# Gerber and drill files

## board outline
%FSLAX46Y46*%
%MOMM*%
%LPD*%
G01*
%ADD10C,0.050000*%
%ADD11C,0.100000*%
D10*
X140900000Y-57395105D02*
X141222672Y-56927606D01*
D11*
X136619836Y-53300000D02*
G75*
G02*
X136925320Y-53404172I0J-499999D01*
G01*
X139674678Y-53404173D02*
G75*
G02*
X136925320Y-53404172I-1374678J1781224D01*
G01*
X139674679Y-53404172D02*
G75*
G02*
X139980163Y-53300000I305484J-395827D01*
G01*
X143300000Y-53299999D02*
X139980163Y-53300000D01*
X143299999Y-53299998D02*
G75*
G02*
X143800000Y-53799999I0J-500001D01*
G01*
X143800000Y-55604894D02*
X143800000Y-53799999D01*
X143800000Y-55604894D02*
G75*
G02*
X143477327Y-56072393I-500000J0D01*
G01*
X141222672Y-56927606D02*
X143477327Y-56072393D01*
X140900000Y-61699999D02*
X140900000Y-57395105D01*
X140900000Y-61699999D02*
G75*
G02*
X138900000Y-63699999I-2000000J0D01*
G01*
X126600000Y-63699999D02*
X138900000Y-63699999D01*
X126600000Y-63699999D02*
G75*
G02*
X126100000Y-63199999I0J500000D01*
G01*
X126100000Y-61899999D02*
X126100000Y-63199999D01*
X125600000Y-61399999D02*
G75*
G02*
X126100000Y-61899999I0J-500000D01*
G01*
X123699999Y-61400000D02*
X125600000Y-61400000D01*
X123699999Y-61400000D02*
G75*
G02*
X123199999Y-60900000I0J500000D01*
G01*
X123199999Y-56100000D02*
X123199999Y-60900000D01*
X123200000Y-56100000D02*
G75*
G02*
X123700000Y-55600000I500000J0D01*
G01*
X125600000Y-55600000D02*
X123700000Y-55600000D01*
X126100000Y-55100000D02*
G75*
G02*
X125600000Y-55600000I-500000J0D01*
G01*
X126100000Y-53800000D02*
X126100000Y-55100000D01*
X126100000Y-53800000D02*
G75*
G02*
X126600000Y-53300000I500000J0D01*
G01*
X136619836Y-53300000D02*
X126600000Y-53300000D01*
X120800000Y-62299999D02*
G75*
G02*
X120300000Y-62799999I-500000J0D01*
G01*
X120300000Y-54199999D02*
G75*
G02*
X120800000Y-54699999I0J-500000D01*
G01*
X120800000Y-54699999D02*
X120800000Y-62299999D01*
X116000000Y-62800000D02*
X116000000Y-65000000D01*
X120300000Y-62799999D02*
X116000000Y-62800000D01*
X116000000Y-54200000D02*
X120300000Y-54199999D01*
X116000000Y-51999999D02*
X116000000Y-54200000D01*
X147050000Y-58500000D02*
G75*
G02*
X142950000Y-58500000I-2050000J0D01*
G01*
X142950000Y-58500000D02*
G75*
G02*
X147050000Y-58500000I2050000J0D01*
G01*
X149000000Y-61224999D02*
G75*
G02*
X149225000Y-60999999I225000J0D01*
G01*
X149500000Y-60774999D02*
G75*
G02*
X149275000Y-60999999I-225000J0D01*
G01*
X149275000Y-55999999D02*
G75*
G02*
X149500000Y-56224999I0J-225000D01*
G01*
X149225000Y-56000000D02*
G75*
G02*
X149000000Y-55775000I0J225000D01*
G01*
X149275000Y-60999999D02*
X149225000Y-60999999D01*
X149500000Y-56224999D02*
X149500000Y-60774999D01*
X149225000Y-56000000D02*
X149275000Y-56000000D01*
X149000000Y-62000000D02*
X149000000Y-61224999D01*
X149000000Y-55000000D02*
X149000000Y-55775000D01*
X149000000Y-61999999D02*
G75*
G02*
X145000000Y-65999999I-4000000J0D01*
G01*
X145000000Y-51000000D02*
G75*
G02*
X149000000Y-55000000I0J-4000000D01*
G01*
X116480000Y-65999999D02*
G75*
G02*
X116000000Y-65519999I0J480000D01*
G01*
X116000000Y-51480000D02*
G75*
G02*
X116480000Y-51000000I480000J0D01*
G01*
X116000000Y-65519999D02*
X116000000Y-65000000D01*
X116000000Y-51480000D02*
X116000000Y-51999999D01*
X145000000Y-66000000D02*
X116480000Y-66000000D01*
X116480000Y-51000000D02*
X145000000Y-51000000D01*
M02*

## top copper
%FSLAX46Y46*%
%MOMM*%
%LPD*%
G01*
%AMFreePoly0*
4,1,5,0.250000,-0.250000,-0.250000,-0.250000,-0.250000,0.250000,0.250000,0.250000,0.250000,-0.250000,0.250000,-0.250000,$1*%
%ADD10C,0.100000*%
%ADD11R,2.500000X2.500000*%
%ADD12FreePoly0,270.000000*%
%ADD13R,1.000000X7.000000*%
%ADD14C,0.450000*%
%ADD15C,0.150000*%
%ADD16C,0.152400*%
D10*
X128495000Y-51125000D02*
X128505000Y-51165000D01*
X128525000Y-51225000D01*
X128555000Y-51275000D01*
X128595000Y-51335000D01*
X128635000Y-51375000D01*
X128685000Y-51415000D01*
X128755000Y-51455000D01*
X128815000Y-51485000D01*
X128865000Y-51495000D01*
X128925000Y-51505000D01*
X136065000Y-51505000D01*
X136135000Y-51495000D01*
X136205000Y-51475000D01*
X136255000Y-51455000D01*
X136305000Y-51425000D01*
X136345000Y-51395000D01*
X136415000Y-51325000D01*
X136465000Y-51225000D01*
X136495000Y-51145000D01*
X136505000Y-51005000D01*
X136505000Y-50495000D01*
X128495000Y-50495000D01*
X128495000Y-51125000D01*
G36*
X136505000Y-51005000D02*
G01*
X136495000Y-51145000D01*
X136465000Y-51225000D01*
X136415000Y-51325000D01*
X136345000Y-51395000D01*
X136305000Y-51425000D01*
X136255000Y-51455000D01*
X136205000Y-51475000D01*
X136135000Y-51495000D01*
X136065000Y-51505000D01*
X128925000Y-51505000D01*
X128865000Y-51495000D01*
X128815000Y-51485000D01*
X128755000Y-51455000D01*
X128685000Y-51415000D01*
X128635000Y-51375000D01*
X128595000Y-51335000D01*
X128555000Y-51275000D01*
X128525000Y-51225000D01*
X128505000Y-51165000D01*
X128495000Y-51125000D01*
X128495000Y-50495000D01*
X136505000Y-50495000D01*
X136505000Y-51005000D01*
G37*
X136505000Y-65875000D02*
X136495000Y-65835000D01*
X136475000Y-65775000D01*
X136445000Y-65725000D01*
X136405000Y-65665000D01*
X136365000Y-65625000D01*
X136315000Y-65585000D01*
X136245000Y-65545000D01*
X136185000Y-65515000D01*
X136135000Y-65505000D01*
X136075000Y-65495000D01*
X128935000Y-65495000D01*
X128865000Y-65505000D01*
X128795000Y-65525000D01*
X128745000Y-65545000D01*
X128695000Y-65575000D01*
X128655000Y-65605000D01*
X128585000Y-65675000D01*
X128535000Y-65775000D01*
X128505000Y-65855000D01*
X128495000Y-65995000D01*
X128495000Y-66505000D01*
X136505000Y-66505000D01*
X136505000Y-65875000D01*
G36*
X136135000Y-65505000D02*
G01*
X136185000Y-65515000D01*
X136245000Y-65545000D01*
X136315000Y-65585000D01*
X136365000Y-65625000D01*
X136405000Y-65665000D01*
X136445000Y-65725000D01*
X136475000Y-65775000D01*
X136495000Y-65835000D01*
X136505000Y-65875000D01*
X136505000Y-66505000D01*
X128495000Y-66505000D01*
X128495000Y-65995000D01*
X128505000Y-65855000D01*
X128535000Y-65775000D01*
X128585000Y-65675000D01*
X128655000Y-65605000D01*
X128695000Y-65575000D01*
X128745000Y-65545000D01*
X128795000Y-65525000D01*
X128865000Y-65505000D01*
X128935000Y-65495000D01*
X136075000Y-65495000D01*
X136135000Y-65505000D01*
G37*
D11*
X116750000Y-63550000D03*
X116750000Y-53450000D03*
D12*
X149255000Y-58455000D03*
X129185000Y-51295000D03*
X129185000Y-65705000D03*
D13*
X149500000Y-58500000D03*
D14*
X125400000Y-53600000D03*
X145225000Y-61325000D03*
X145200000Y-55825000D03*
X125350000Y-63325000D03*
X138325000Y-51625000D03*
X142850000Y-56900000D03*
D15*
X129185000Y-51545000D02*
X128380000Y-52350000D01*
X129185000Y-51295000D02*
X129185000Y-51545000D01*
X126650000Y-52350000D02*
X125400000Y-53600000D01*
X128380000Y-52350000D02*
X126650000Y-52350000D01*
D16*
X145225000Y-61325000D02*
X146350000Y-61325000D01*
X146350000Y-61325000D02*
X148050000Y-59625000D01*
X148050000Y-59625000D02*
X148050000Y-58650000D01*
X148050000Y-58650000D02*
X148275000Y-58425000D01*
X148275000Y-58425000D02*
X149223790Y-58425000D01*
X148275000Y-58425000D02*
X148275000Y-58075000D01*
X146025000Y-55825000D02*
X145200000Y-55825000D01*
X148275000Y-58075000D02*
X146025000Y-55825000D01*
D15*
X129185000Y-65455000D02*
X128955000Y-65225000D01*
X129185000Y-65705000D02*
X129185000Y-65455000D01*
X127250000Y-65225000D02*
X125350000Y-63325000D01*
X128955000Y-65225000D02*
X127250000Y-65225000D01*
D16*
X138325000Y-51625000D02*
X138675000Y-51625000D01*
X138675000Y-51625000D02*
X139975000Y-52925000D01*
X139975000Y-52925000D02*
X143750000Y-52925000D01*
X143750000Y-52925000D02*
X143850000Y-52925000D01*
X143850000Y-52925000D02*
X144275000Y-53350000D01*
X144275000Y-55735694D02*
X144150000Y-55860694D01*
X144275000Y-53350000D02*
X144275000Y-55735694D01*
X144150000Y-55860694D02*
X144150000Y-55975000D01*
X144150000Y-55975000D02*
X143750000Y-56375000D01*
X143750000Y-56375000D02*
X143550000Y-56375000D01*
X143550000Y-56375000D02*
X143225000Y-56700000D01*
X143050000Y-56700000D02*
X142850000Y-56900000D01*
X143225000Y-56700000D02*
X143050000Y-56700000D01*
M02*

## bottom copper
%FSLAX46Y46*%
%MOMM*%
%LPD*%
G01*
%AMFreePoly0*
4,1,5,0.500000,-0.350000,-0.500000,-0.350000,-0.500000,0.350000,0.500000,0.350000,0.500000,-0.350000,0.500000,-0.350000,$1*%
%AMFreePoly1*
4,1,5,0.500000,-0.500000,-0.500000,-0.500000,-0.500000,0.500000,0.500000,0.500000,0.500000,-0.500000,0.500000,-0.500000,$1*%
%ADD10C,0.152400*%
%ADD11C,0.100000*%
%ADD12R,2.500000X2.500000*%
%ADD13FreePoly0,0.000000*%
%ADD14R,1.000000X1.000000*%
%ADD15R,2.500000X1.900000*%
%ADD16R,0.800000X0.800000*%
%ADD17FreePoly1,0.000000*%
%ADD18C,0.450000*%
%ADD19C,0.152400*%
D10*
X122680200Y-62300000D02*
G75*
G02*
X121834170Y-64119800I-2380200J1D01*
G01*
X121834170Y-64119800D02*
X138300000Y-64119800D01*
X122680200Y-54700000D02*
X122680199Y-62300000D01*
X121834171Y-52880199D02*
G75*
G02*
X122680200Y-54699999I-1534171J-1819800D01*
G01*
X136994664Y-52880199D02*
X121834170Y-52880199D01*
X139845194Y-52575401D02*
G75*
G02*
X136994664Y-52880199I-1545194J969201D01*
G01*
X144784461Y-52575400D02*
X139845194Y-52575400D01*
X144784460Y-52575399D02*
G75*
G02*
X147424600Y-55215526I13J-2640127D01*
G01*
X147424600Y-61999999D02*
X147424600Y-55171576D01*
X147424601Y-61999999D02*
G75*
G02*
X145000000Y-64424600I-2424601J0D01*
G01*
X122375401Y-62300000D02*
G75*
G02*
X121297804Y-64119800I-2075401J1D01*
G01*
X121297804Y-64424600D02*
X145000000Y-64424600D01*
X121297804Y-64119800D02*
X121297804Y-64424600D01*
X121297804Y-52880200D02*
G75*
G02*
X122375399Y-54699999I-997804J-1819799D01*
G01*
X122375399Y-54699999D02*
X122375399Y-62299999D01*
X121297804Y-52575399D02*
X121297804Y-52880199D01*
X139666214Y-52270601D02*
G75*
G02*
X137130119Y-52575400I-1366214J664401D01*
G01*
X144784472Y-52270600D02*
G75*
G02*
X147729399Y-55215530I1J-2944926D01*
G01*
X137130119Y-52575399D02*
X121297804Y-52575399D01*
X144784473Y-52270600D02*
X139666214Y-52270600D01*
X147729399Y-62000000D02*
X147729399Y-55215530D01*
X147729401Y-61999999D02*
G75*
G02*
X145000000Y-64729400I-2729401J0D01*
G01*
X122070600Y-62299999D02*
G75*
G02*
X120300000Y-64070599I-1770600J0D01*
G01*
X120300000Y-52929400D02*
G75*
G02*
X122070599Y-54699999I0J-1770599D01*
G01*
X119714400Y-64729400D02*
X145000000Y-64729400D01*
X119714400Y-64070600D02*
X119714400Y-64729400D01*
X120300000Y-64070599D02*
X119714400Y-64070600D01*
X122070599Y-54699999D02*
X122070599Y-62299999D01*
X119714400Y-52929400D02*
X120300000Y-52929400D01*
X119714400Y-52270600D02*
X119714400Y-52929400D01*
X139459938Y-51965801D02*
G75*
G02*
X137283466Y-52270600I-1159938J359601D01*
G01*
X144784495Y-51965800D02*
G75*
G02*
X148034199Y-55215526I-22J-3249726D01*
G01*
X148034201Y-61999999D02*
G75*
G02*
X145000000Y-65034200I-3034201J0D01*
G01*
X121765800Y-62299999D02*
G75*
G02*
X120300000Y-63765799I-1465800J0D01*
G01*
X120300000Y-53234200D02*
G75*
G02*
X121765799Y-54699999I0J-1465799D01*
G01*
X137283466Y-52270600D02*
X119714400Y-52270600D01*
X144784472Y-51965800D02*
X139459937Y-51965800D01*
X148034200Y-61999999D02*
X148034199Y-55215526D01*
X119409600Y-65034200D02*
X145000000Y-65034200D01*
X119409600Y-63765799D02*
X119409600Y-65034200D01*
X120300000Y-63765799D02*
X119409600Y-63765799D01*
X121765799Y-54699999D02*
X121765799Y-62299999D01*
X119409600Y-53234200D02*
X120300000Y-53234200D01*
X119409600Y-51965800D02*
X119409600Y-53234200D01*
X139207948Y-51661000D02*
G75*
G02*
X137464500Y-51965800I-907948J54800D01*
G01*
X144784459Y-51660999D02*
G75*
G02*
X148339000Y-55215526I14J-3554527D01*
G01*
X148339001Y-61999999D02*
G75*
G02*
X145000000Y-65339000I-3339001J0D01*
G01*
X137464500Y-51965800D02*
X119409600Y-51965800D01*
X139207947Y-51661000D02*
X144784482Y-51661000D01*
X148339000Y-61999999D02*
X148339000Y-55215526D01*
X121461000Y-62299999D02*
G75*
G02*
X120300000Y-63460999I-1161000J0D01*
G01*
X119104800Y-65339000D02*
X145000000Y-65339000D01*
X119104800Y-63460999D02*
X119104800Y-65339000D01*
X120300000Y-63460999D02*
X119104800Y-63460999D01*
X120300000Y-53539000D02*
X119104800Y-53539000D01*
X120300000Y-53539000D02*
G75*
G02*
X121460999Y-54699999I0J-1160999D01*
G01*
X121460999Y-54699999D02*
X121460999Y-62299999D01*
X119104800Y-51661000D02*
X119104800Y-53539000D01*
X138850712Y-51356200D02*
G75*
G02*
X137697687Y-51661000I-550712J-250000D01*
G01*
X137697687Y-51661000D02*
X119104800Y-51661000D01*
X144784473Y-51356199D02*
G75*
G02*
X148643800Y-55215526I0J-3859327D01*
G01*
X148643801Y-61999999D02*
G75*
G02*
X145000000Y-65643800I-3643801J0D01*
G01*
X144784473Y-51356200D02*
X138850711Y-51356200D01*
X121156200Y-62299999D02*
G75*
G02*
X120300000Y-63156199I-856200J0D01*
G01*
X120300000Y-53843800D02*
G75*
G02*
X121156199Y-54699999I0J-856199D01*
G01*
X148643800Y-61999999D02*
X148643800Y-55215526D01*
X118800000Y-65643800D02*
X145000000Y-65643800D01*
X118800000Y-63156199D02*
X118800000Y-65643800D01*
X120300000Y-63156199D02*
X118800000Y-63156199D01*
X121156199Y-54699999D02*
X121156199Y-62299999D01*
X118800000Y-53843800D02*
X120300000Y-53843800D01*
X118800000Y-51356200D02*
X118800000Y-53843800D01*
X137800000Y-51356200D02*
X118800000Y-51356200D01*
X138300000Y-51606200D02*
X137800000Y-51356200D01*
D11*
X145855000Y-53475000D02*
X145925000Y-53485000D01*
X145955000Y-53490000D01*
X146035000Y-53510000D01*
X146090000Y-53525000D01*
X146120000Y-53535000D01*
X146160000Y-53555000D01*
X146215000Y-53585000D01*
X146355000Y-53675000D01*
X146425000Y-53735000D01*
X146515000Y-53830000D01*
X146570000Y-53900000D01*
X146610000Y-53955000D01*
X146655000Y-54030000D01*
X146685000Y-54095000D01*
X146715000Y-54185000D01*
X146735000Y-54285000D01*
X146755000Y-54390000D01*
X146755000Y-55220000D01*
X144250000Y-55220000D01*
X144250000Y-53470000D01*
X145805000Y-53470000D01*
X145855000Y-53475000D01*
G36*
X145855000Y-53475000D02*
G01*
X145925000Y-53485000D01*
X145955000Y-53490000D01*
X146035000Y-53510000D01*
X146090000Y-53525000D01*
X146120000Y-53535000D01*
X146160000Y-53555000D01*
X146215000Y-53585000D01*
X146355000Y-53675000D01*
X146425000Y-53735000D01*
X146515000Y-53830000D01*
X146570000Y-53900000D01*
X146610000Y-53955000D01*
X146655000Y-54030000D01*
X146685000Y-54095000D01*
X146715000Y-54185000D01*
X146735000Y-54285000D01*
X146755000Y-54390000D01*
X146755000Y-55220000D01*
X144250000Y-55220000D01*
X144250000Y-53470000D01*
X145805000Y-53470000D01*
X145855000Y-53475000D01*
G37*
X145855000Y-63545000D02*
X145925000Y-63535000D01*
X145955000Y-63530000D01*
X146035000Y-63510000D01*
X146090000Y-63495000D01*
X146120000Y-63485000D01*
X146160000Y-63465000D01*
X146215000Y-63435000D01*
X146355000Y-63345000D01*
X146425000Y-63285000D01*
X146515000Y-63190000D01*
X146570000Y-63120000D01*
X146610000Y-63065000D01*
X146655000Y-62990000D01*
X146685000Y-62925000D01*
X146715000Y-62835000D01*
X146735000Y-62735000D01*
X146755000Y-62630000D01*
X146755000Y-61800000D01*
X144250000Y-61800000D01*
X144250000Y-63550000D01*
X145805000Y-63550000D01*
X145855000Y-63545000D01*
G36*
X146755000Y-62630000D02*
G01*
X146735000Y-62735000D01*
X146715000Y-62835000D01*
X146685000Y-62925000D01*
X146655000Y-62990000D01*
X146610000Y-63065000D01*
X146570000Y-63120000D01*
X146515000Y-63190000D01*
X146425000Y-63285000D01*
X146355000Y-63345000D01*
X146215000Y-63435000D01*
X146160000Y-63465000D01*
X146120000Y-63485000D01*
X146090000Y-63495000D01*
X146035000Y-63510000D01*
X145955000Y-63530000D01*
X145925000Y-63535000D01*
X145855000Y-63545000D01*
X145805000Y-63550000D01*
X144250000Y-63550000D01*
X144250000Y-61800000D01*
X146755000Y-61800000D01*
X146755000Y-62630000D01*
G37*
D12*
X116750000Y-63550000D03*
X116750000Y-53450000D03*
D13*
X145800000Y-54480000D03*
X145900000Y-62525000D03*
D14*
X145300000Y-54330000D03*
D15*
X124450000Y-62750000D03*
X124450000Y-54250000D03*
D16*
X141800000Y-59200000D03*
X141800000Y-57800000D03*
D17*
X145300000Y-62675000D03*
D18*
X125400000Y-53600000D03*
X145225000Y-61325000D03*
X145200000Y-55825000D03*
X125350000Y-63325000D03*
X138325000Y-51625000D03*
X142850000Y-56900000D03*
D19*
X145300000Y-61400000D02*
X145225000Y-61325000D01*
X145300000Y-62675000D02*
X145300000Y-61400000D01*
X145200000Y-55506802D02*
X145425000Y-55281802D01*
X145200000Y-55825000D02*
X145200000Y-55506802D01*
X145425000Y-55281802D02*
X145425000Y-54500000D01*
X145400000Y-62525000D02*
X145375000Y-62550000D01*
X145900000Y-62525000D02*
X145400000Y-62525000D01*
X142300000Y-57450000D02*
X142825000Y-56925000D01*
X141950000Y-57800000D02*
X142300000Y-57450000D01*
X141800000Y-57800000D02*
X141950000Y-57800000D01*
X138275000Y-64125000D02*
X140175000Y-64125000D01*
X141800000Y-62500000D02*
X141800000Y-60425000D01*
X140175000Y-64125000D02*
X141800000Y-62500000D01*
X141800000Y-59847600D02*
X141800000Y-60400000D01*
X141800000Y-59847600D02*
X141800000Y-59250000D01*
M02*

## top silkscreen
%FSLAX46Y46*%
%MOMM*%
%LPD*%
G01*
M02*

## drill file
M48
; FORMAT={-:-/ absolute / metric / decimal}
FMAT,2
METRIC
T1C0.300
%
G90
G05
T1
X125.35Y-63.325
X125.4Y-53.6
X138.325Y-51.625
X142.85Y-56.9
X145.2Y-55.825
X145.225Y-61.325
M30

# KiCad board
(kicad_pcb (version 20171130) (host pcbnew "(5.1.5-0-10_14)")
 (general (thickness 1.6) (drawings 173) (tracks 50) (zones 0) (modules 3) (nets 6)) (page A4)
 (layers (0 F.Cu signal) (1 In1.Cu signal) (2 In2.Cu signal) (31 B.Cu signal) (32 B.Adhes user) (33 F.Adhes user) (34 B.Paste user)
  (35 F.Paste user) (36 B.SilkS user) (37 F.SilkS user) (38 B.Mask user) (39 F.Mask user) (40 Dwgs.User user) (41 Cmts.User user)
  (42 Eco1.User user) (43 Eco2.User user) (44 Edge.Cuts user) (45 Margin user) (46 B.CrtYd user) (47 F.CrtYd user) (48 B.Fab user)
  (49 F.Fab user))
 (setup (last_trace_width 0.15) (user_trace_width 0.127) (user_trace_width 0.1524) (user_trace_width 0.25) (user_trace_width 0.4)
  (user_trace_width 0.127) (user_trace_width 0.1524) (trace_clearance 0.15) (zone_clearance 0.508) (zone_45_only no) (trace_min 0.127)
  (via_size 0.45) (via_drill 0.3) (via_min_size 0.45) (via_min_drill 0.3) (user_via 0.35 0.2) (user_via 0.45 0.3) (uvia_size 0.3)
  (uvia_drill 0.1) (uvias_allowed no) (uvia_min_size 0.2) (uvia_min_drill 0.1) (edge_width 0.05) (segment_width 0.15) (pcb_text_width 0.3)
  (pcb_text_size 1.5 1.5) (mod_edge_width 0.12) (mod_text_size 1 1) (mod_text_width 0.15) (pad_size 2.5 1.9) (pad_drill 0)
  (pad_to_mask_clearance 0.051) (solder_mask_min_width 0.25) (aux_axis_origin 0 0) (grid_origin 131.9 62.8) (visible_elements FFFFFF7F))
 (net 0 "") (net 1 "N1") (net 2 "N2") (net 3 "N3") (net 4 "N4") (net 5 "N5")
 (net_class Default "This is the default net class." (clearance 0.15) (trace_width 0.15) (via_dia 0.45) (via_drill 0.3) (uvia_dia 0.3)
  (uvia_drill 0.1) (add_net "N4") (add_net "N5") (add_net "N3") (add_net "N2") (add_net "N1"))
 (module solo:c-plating (layer F.Cu) (at 116.9 53.35)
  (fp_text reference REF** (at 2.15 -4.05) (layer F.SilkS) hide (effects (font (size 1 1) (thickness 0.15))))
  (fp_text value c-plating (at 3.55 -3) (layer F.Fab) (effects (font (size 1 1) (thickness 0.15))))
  (pad 1 smd rect (at -0.15 10.2) (size 2.5 2.5) (layers B.Cu B.Mask))
  (pad 1 smd rect (at -0.15 0.1) (size 2.5 2.5) (layers B.Cu B.Mask))
  (pad 2 smd rect (at -0.15 10.2) (size 2.5 2.5) (layers F.Cu F.Mask))
  (pad 1 smd rect (at -0.15 0.1) (size 2.5 2.5) (layers F.Cu F.Mask)))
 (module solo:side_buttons (layer B.Cu) (at 149.525 58.075)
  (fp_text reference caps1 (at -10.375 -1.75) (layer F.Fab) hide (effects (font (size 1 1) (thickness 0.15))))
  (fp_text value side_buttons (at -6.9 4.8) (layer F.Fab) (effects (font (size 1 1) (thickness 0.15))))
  (fp_poly
   (pts (xy -21.03 -6.95) (xy -21.02 -6.91) (xy -21 -6.85) (xy -20.97 -6.8) (xy -20.93 -6.74) (xy -20.89 -6.7) (xy -20.84 -6.66)
    (xy -20.77 -6.62) (xy -20.71 -6.59) (xy -20.66 -6.58) (xy -20.6 -6.57) (xy -13.46 -6.57) (xy -13.39 -6.58) (xy -13.32 -6.6)
    (xy -13.27 -6.62) (xy -13.22 -6.65) (xy -13.18 -6.68) (xy -13.11 -6.75) (xy -13.06 -6.85) (xy -13.03 -6.93) (xy -13.02 -7.07)
    (xy -13.02 -7.58) (xy -21.03 -7.58))
   (layer F.Cu) (width 0.1))
  (fp_poly
   (pts (xy -13.02 7.8) (xy -13.03 7.76) (xy -13.05 7.7) (xy -13.08 7.65) (xy -13.12 7.59) (xy -13.16 7.55) (xy -13.21 7.51)
    (xy -13.28 7.47) (xy -13.34 7.44) (xy -13.39 7.43) (xy -13.45 7.42) (xy -20.59 7.42) (xy -20.66 7.43) (xy -20.73 7.45) (xy -20.78 7.47)
    (xy -20.83 7.5) (xy -20.87 7.53) (xy -20.94 7.6) (xy -20.99 7.7) (xy -21.02 7.78) (xy -21.03 7.92) (xy -21.03 8.43) (xy -13.02 8.43))
   (layer F.Cu) (width 0.1))
  (pad 3 smd custom (at -0.27 0.38 270) (size 0.5 0.5) (layers F.Cu) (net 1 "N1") (solder_mask_margin 0.01) (zone_connect 0)
   (options (clearance outline) (anchor rect)) (primitives))
  (pad 2 smd custom (at -20.34 -6.78 270) (size 0.5 0.5) (layers F.Cu) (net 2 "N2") (solder_mask_margin 0.01) (zone_connect 0)
   (options (clearance outline) (anchor rect)) (primitives))
  (pad 1 smd custom (at -20.34 7.63 270) (size 0.5 0.5) (layers F.Cu) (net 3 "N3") (solder_mask_margin 0.01) (zone_connect 0)
   (options (clearance outline) (anchor rect)) (primitives))
  (pad 3 smd rect (at -0.025 0.425 270) (size 7 1) (layers F.Cu F.Mask) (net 1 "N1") (solder_mask_margin 0.01)))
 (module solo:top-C (layer B.Cu) (at 114.8 58.375)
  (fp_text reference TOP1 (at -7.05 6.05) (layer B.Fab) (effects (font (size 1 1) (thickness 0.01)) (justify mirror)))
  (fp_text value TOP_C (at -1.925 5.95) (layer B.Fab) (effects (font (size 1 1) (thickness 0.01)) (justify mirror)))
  (fp_poly
   (pts (xy 31.055 -4.9) (xy 31.125 -4.89) (xy 31.155 -4.885) (xy 31.235 -4.865) (xy 31.29 -4.85) (xy 31.32 -4.84) (xy 31.36 -4.82)
    (xy 31.415 -4.79) (xy 31.555 -4.7) (xy 31.625 -4.64) (xy 31.715 -4.545) (xy 31.77 -4.475) (xy 31.81 -4.42) (xy 31.855 -4.345)
    (xy 31.885 -4.28) (xy 31.915 -4.19) (xy 31.935 -4.09) (xy 31.955 -3.985) (xy 31.955 -3.155) (xy 29.45 -3.155) (xy 29.45 -4.905)
    (xy 31.005 -4.905))
   (layer B.Cu) (width 0.1))
  (fp_poly
   (pts (xy 31.055 5.17) (xy 31.125 5.16) (xy 31.155 5.155) (xy 31.235 5.135) (xy 31.29 5.12) (xy 31.32 5.11) (xy 31.36 5.09)
    (xy 31.415 5.06) (xy 31.555 4.97) (xy 31.625 4.91) (xy 31.715 4.815) (xy 31.77 4.745) (xy 31.81 4.69) (xy 31.855 4.615) (xy 31.885 4.55)
    (xy 31.915 4.46) (xy 31.935 4.36) (xy 31.955 4.255) (xy 31.955 3.425) (xy 29.45 3.425) (xy 29.45 5.175) (xy 31.005 5.175))
   (layer B.Cu) (width 0.1))
  (pad 9 smd custom (at 31 -3.895) (size 1 0.7) (layers B.Cu B.Paste B.Mask) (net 1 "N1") (solder_paste_margin_ratio -0.05) (zone_connect 0)
   (options (clearance outline) (anchor rect)) (primitives))
  (pad 9 smd custom (at 31.1 4.15) (size 1 0.7) (layers B.Cu B.Paste B.Mask) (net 1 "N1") (solder_paste_margin_ratio -0.05) (zone_connect 0)
   (options (clearance outline) (anchor rect)) (primitives))
  (pad 9 smd rect (at 30.5 -4.045) (size 1 1) (layers B.Cu B.Paste B.Mask) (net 1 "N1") (solder_paste_margin_ratio -0.05))
  (pad 5 smd rect (at 9.65 4.375) (size 2.5 1.9) (layers B.Cu B.Paste B.Mask) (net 3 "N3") (solder_paste_margin_ratio -0.25))
  (pad 6 smd rect (at 9.65 -4.125) (size 2.5 1.9) (layers B.Cu B.Paste B.Mask) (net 2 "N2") (solder_paste_margin_ratio -0.25))
  (pad 7 smd rect (at 27 0.825) (size 0.8 0.8) (layers B.Cu B.Paste B.Mask) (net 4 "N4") (solder_paste_margin_ratio -0.2))
  (pad 8 smd rect (at 27 -0.575) (size 0.8 0.8) (layers B.Cu B.Paste B.Mask) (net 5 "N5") (solder_paste_margin_ratio -0.2))
  (pad 9 smd custom (at 30.5 4.3) (size 1 1) (layers B.Cu B.Paste B.Mask) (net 1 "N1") (solder_paste_margin_ratio -0.05) (zone_connect 0)
   (options (clearance outline) (anchor rect)) (primitives)))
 (gr_line (start 140.9 57.395105) (end 141.222672 56.927606) (layer Edge.Cuts) (width 0.05))
 (gr_arc (start 120.3 62.299999) (end 121.83417 64.1198) (angle -49.86765021) (layer B.Cu) (width 0.1524))
 (gr_line (start 121.83417 64.1198) (end 138.3 64.1198) (layer B.Cu) (width 0.1524))
 (gr_line (start 122.6802 54.7) (end 122.680199 62.3) (layer B.Cu) (width 0.1524))
 (gr_arc (start 120.3 54.699999) (end 122.6802 54.699999) (angle -49.86765021) (layer B.Cu) (width 0.1524))
 (gr_line (start 136.994664 52.880199) (end 121.83417 52.880199) (layer B.Cu) (width 0.1524))
 (gr_arc (start 138.3 51.6062) (end 136.994664 52.880199) (angle -103.59866) (layer B.Cu) (width 0.1524))
 (gr_line (start 144.784461 52.5754) (end 139.845194 52.5754) (layer B.Cu) (width 0.1524))
 (gr_arc (start 144.784473 55.215526) (end 147.4246 55.215526) (angle -90.00027385) (layer B.Cu) (width 0.1524))
 (gr_line (start 147.4246 61.999999) (end 147.4246 55.171576) (layer B.Cu) (width 0.1524))
 (gr_arc (start 145 61.999999) (end 145 64.4246) (angle -90) (layer B.Cu) (width 0.1524))
 (gr_arc (start 120.3 62.299999) (end 121.297804 64.1198) (angle -61.26385234) (layer B.Cu) (width 0.1524))
 (gr_line (start 121.297804 64.4246) (end 145 64.4246) (layer B.Cu) (width 0.1524))
 (gr_line (start 121.297804 64.1198) (end 121.297804 64.4246) (layer B.Cu) (width 0.1524))
 (gr_arc (start 120.3 54.699999) (end 122.375399 54.699999) (angle -61.26385234) (layer B.Cu) (width 0.1524))
 (gr_line (start 122.375399 54.699999) (end 122.375399 62.299999) (layer B.Cu) (width 0.1524))
 (gr_line (start 121.297804 52.575399) (end 121.297804 52.880199) (layer B.Cu) (width 0.1524))
 (gr_arc (start 138.3 51.6062) (end 137.130119 52.5754) (angle -114.4255887) (layer B.Cu) (width 0.1524))
 (gr_arc (start 144.784473 55.215526) (end 147.729399 55.21553) (angle -90.0000935) (layer B.Cu) (width 0.1524))
 (gr_line (start 137.130119 52.575399) (end 121.297804 52.575399) (layer B.Cu) (width 0.1524))
 (gr_line (start 144.784473 52.2706) (end 139.666214 52.2706) (layer B.Cu) (width 0.1524))
 (gr_line (start 147.729399 62) (end 147.729399 55.21553) (layer B.Cu) (width 0.1524))
 (gr_arc (start 145 61.999999) (end 145 64.7294) (angle -90) (layer B.Cu) (width 0.1524))
 (gr_arc (start 120.3 62.299999) (end 120.3 64.070599) (angle -89.99998951) (layer B.Cu) (width 0.1524))
 (gr_arc (start 120.3 54.699999) (end 122.070599 54.699999) (angle -90) (layer B.Cu) (width 0.1524))
 (gr_line (start 119.7144 64.7294) (end 145 64.7294) (layer B.Cu) (width 0.1524))
 (gr_line (start 119.7144 64.0706) (end 119.7144 64.7294) (layer B.Cu) (width 0.1524))
 (gr_line (start 120.3 64.070599) (end 119.7144 64.0706) (layer B.Cu) (width 0.1524))
 (gr_line (start 122.070599 54.699999) (end 122.070599 62.299999) (layer B.Cu) (width 0.1524))
 (gr_line (start 119.7144 52.9294) (end 120.3 52.9294) (layer B.Cu) (width 0.1524))
 (gr_line (start 119.7144 52.2706) (end 119.7144 52.9294) (layer B.Cu) (width 0.1524))
 (gr_arc (start 138.3 51.6062) (end 137.283466 52.2706) (angle -129.6073052) (layer B.Cu) (width 0.1524))
 (gr_arc (start 144.784473 55.215526) (end 148.034199 55.215526) (angle -89.99961615) (layer B.Cu) (width 0.1524))
 (gr_arc (start 145 61.999999) (end 145 65.0342) (angle -90) (layer B.Cu) (width 0.1524))
 (gr_arc (start 120.3 62.299999) (end 120.3 63.765799) (angle -90) (layer B.Cu) (width 0.1524))
 (gr_arc (start 120.3 54.699999) (end 121.765799 54.699999) (angle -90) (layer B.Cu) (width 0.1524))
 (gr_line (start 137.283466 52.2706) (end 119.7144 52.2706) (layer B.Cu) (width 0.1524))
 (gr_line (start 144.784472 51.9658) (end 139.459937 51.9658) (layer B.Cu) (width 0.1524))
 (gr_line (start 148.0342 61.999999) (end 148.034199 55.215526) (layer B.Cu) (width 0.1524))
 (gr_line (start 119.4096 65.0342) (end 145 65.0342) (layer B.Cu) (width 0.1524))
 (gr_line (start 119.4096 63.765799) (end 119.4096 65.0342) (layer B.Cu) (width 0.1524))
 (gr_line (start 120.3 63.765799) (end 119.4096 63.765799) (layer B.Cu) (width 0.1524))
 (gr_line (start 121.765799 54.699999) (end 121.765799 62.299999) (layer B.Cu) (width 0.1524))
 (gr_line (start 119.4096 53.2342) (end 120.3 53.2342) (layer B.Cu) (width 0.1524))
 (gr_line (start 119.4096 51.9658) (end 119.4096 53.2342) (layer B.Cu) (width 0.1524))
 (gr_arc (start 138.3 51.6062) (end 137.4645 51.9658) (angle -153.2589579) (layer B.Cu) (width 0.1524))
 (gr_arc (start 144.784473 55.215526) (end 148.339 55.215526) (angle -90.00022865) (layer B.Cu) (width 0.1524))
 (gr_arc (start 145 61.999999) (end 145 65.339) (angle -90) (layer B.Cu) (width 0.1524))
 (gr_line (start 137.4645 51.9658) (end 119.4096 51.9658) (layer B.Cu) (width 0.1524))
 (gr_line (start 139.207947 51.661) (end 144.784482 51.661) (layer B.Cu) (width 0.1524))
 (gr_line (start 148.339 61.999999) (end 148.339 55.215526) (layer B.Cu) (width 0.1524))
 (gr_arc (start 120.3 62.299999) (end 120.3 63.460999) (angle -90) (layer B.Cu) (width 0.1524))
 (gr_line (start 119.1048 65.339) (end 145 65.339) (layer B.Cu) (width 0.1524))
 (gr_line (start 119.1048 63.460999) (end 119.1048 65.339) (layer B.Cu) (width 0.1524))
 (gr_line (start 120.3 63.460999) (end 119.1048 63.460999) (layer B.Cu) (width 0.1524))
 (gr_line (start 120.3 53.539) (end 119.1048 53.539) (layer B.Cu) (width 0.1524))
 (gr_arc (start 120.3 54.699999) (end 121.460999 54.699999) (angle -90) (layer B.Cu) (width 0.1524))
 (gr_line (start 121.460999 54.699999) (end 121.460999 62.299999) (layer B.Cu) (width 0.1524))
 (gr_line (start 119.1048 51.661) (end 119.1048 53.539) (layer B.Cu) (width 0.1524))
 (gr_arc (start 138.3 51.6062) (end 137.697687 51.661) (angle -199.2174543) (layer B.Cu) (width 0.1524))
 (gr_line (start 137.697687 51.661) (end 119.1048 51.661) (layer B.Cu) (width 0.1524))
 (gr_arc (start 144.784473 55.215526) (end 148.6438 55.215526) (angle -90) (layer B.Cu) (width 0.1524))
 (gr_arc (start 145 61.999999) (end 145 65.6438) (angle -90) (layer B.Cu) (width 0.1524))
 (gr_line (start 144.784473 51.3562) (end 138.850711 51.3562) (layer B.Cu) (width 0.1524))
 (gr_arc (start 120.3 62.299999) (end 120.3 63.156199) (angle -90) (layer B.Cu) (width 0.1524))
 (gr_arc (start 120.3 54.699999) (end 121.156199 54.699999) (angle -90) (layer B.Cu) (width 0.1524))
 (gr_line (start 148.6438 61.999999) (end 148.6438 55.215526) (layer B.Cu) (width 0.1524))
 (gr_line (start 118.8 65.6438) (end 145 65.6438) (layer B.Cu) (width 0.1524))
 (gr_line (start 118.8 63.156199) (end 118.8 65.6438) (layer B.Cu) (width 0.1524))
 (gr_line (start 120.3 63.156199) (end 118.8 63.156199) (layer B.Cu) (width 0.1524))
 (gr_line (start 121.156199 54.699999) (end 121.156199 62.299999) (layer B.Cu) (width 0.1524))
 (gr_line (start 118.8 53.8438) (end 120.3 53.8438) (layer B.Cu) (width 0.1524))
 (gr_line (start 118.8 51.3562) (end 118.8 53.8438) (layer B.Cu) (width 0.1524))
 (gr_line (start 137.8 51.3562) (end 118.8 51.3562) (layer B.Cu) (width 0.1524))
 (gr_line (start 138.3 51.6062) (end 137.8 51.3562) (layer B.Cu) (width 0.1524))
 (gr_arc (start 136.619836 53.799999) (end 136.92532 53.404172) (angle -37.6595652) (layer Edge.Cuts) (width 0.1))
 (gr_arc (start 138.3 51.622949) (end 136.92532 53.404172) (angle -75.31913041) (layer Edge.Cuts) (width 0.1))
 (gr_arc (start 139.980163 53.799999) (end 139.980163 53.3) (angle -37.6595652) (layer Edge.Cuts) (width 0.1))
 (gr_line (start 143.3 53.299999) (end 139.980163 53.3) (layer Edge.Cuts) (width 0.1))
 (gr_arc (start 143.299999 53.799999) (end 143.8 53.799999) (angle -90) (layer Edge.Cuts) (width 0.1))
 (gr_line (start 143.8 55.604894) (end 143.8 53.799999) (layer Edge.Cuts) (width 0.1))
 (gr_arc (start 143.3 55.604894) (end 143.477327 56.072393) (angle -69.22774532) (layer Edge.Cuts) (width 0.1))
 (gr_line (start 141.222672 56.927606) (end 143.477327 56.072393) (layer Edge.Cuts) (width 0.1))
 (gr_line (start 140.9 61.699999) (end 140.9 57.395105) (layer Edge.Cuts) (width 0.1))
 (gr_arc (start 138.9 61.699999) (end 138.9 63.699999) (angle -90) (layer Edge.Cuts) (width 0.1))
 (gr_line (start 126.6 63.699999) (end 138.9 63.699999) (layer Edge.Cuts) (width 0.1))
 (gr_arc (start 126.6 63.199999) (end 126.1 63.199999) (angle -90) (layer Edge.Cuts) (width 0.1))
 (gr_line (start 126.1 61.899999) (end 126.1 63.199999) (layer Edge.Cuts) (width 0.1))
 (gr_arc (start 125.6 61.899999) (end 126.1 61.899999) (angle -90) (layer Edge.Cuts) (width 0.1))
 (gr_line (start 123.699999 61.4) (end 125.6 61.4) (layer Edge.Cuts) (width 0.1))
 (gr_arc (start 123.699999 60.9) (end 123.199999 60.9) (angle -90) (layer Edge.Cuts) (width 0.1))
 (gr_line (start 123.199999 56.1) (end 123.199999 60.9) (layer Edge.Cuts) (width 0.1))
 (gr_arc (start 123.7 56.1) (end 123.7 55.6) (angle -90) (layer Edge.Cuts) (width 0.1))
 (gr_line (start 125.6 55.6) (end 123.7 55.6) (layer Edge.Cuts) (width 0.1))
 (gr_arc (start 125.6 55.1) (end 125.6 55.6) (angle -90) (layer Edge.Cuts) (width 0.1))
 (gr_line (start 126.1 53.8) (end 126.1 55.1) (layer Edge.Cuts) (width 0.1))
 (gr_arc (start 126.6 53.8) (end 126.6 53.3) (angle -90) (layer Edge.Cuts) (width 0.1))
 (gr_line (start 136.619836 53.3) (end 126.6 53.3) (layer Edge.Cuts) (width 0.1))
 (gr_arc (start 120.3 62.299999) (end 120.3 62.799999) (angle -90) (layer Edge.Cuts) (width 0.1))
 (gr_arc (start 120.3 54.699999) (end 120.8 54.699999) (angle -90) (layer Edge.Cuts) (width 0.1))
 (gr_line (start 120.8 54.699999) (end 120.8 62.299999) (layer Edge.Cuts) (width 0.1))
 (gr_line (start 116 62.8) (end 116 65) (layer Edge.Cuts) (width 0.1))
 (gr_line (start 120.3 62.799999) (end 116 62.8) (layer Edge.Cuts) (width 0.1))
 (gr_line (start 116 54.2) (end 120.3 54.199999) (layer Edge.Cuts) (width 0.1))
 (gr_line (start 116 51.999999) (end 116 54.2) (layer Edge.Cuts) (width 0.1))
 (gr_circle (center 145 58.5) (end 147.05 58.5) (layer Edge.Cuts) (width 0.1))
 (gr_arc (start 149.225 61.224999) (end 149.225 60.999999) (angle -90) (layer Edge.Cuts) (width 0.1))
 (gr_arc (start 149.275 60.774999) (end 149.275 60.999999) (angle -90) (layer Edge.Cuts) (width 0.1))
 (gr_arc (start 149.275 56.224999) (end 149.5 56.224999) (angle -90) (layer Edge.Cuts) (width 0.1))
 (gr_arc (start 149.225 55.775) (end 149 55.775) (angle -90) (layer Edge.Cuts) (width 0.1))
 (gr_line (start 149.275 60.999999) (end 149.225 60.999999) (layer Edge.Cuts) (width 0.1))
 (gr_line (start 149.5 56.224999) (end 149.5 60.774999) (layer Edge.Cuts) (width 0.1))
 (gr_line (start 149.225 56) (end 149.275 56) (layer Edge.Cuts) (width 0.1))
 (gr_line (start 149 62) (end 149 61.224999) (layer Edge.Cuts) (width 0.1))
 (gr_line (start 149 55) (end 149 55.775) (layer Edge.Cuts) (width 0.1))
 (gr_arc (start 145 61.999999) (end 145 65.999999) (angle -90) (layer Edge.Cuts) (width 0.1))
 (gr_arc (start 145 55) (end 149 55) (angle -90) (layer Edge.Cuts) (width 0.1))
 (gr_arc (start 116.48 65.519999) (end 116 65.519999) (angle -90) (layer Edge.Cuts) (width 0.1))
 (gr_arc (start 116.48 51.48) (end 116.48 51) (angle -90) (layer Edge.Cuts) (width 0.1))
 (gr_line (start 116 65.519999) (end 116 65) (layer Edge.Cuts) (width 0.1))
 (gr_line (start 116 51.48) (end 116 51.999999) (layer Edge.Cuts) (width 0.1))
 (gr_line (start 145 66) (end 116.48 66) (layer Edge.Cuts) (width 0.1))
 (gr_line (start 116.48 51) (end 145 51) (layer Edge.Cuts) (width 0.1))
 (segment (start 129.185 51.545) (end 128.38 52.35) (width 0.15) (layer F.Cu) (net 2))
 (segment (start 129.185 51.295) (end 129.185 51.545) (width 0.15) (layer F.Cu) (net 2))
 (via (at 125.4 53.6) (size 0.45) (drill 0.3) (layers F.Cu B.Cu) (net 2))
 (segment (start 126.65 52.35) (end 125.4 53.6) (width 0.15) (layer F.Cu) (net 2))
 (segment (start 128.38 52.35) (end 126.65 52.35) (width 0.15) (layer F.Cu) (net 2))
 (via (at 145.225 61.325) (size 0.45) (drill 0.3) (layers F.Cu B.Cu) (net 1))
 (segment (start 145.3 61.4) (end 145.225 61.325) (width 0.1524) (layer B.Cu) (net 1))
 (segment (start 145.3 62.675) (end 145.3 61.4) (width 0.1524) (layer B.Cu) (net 1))
 (segment (start 145.225 61.325) (end 146.35 61.325) (width 0.1524) (layer F.Cu) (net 1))
 (segment (start 146.35 61.325) (end 148.05 59.625) (width 0.1524) (layer F.Cu) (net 1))
 (segment (start 148.05 59.625) (end 148.05 58.65) (width 0.1524) (layer F.Cu) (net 1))
 (segment (start 148.05 58.65) (end 148.275 58.425) (width 0.1524) (layer F.Cu) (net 1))
 (segment (start 148.275 58.425) (end 149.22379 58.425) (width 0.1524) (layer F.Cu) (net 1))
 (segment (start 148.275 58.425) (end 148.275 58.075) (width 0.1524) (layer F.Cu) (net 1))
 (via (at 145.2 55.825) (size 0.45) (drill 0.3) (layers F.Cu B.Cu) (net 1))
 (segment (start 146.025 55.825) (end 145.2 55.825) (width 0.1524) (layer F.Cu) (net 1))
 (segment (start 148.275 58.075) (end 146.025 55.825) (width 0.1524) (layer F.Cu) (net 1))
 (segment (start 145.2 55.506802) (end 145.425 55.281802) (width 0.1524) (layer B.Cu) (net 1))
 (segment (start 145.2 55.825) (end 145.2 55.506802) (width 0.1524) (layer B.Cu) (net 1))
 (segment (start 145.425 55.281802) (end 145.425 54.5) (width 0.1524) (layer B.Cu) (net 1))
 (segment (start 145.4 62.525) (end 145.375 62.55) (width 0.1524) (layer B.Cu) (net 1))
 (segment (start 145.9 62.525) (end 145.4 62.525) (width 0.1524) (layer B.Cu) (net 1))
 (segment (start 129.185 65.455) (end 128.955 65.225) (width 0.15) (layer F.Cu) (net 3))
 (segment (start 129.185 65.705) (end 129.185 65.455) (width 0.15) (layer F.Cu) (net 3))
 (via (at 125.35 63.325) (size 0.45) (drill 0.3) (layers F.Cu B.Cu) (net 3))
 (segment (start 127.25 65.225) (end 125.35 63.325) (width 0.15) (layer F.Cu) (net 3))
 (segment (start 128.955 65.225) (end 127.25 65.225) (width 0.15) (layer F.Cu) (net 3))
 (via (at 138.325 51.625) (size 0.45) (drill 0.3) (layers F.Cu B.Cu) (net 5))
 (segment (start 138.325 51.625) (end 138.675 51.625) (width 0.1524) (layer F.Cu) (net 5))
 (segment (start 138.675 51.625) (end 139.975 52.925) (width 0.1524) (layer F.Cu) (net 5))
 (segment (start 139.975 52.925) (end 143.75 52.925) (width 0.1524) (layer F.Cu) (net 5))
 (segment (start 143.75 52.925) (end 143.85 52.925) (width 0.1524) (layer F.Cu) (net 5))
 (segment (start 143.85 52.925) (end 144.275 53.35) (width 0.1524) (layer F.Cu) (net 5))
 (segment (start 144.275 55.735694) (end 144.15 55.860694) (width 0.1524) (layer F.Cu) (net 5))
 (segment (start 144.275 53.35) (end 144.275 55.735694) (width 0.1524) (layer F.Cu) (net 5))
 (segment (start 144.15 55.860694) (end 144.15 55.975) (width 0.1524) (layer F.Cu) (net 5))
 (segment (start 144.15 55.975) (end 143.75 56.375) (width 0.1524) (layer F.Cu) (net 5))
 (segment (start 143.75 56.375) (end 143.55 56.375) (width 0.1524) (layer F.Cu) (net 5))
 (segment (start 143.55 56.375) (end 143.225 56.7) (width 0.1524) (layer F.Cu) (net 5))
 (via (at 142.85 56.9) (size 0.45) (drill 0.3) (layers F.Cu B.Cu) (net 5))
 (segment (start 143.05 56.7) (end 142.85 56.9) (width 0.1524) (layer F.Cu) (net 5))
 (segment (start 143.225 56.7) (end 143.05 56.7) (width 0.1524) (layer F.Cu) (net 5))
 (segment (start 142.3 57.45) (end 142.825 56.925) (width 0.1524) (layer B.Cu) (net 5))
 (segment (start 141.95 57.8) (end 142.3 57.45) (width 0.1524) (layer B.Cu) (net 5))
 (segment (start 141.8 57.8) (end 141.95 57.8) (width 0.1524) (layer B.Cu) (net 5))
 (segment (start 138.275 64.125) (end 140.175 64.125) (width 0.1524) (layer B.Cu) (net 4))
 (segment (start 141.8 62.5) (end 141.8 60.425) (width 0.1524) (layer B.Cu) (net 4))
 (segment (start 140.175 64.125) (end 141.8 62.5) (width 0.1524) (layer B.Cu) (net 4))
 (segment (start 141.8 59.8476) (end 141.8 60.4) (width 0.1524) (layer B.Cu) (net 4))
 (segment (start 141.8 59.8476) (end 141.8 59.25) (width 0.1524) (layer B.Cu) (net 4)))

